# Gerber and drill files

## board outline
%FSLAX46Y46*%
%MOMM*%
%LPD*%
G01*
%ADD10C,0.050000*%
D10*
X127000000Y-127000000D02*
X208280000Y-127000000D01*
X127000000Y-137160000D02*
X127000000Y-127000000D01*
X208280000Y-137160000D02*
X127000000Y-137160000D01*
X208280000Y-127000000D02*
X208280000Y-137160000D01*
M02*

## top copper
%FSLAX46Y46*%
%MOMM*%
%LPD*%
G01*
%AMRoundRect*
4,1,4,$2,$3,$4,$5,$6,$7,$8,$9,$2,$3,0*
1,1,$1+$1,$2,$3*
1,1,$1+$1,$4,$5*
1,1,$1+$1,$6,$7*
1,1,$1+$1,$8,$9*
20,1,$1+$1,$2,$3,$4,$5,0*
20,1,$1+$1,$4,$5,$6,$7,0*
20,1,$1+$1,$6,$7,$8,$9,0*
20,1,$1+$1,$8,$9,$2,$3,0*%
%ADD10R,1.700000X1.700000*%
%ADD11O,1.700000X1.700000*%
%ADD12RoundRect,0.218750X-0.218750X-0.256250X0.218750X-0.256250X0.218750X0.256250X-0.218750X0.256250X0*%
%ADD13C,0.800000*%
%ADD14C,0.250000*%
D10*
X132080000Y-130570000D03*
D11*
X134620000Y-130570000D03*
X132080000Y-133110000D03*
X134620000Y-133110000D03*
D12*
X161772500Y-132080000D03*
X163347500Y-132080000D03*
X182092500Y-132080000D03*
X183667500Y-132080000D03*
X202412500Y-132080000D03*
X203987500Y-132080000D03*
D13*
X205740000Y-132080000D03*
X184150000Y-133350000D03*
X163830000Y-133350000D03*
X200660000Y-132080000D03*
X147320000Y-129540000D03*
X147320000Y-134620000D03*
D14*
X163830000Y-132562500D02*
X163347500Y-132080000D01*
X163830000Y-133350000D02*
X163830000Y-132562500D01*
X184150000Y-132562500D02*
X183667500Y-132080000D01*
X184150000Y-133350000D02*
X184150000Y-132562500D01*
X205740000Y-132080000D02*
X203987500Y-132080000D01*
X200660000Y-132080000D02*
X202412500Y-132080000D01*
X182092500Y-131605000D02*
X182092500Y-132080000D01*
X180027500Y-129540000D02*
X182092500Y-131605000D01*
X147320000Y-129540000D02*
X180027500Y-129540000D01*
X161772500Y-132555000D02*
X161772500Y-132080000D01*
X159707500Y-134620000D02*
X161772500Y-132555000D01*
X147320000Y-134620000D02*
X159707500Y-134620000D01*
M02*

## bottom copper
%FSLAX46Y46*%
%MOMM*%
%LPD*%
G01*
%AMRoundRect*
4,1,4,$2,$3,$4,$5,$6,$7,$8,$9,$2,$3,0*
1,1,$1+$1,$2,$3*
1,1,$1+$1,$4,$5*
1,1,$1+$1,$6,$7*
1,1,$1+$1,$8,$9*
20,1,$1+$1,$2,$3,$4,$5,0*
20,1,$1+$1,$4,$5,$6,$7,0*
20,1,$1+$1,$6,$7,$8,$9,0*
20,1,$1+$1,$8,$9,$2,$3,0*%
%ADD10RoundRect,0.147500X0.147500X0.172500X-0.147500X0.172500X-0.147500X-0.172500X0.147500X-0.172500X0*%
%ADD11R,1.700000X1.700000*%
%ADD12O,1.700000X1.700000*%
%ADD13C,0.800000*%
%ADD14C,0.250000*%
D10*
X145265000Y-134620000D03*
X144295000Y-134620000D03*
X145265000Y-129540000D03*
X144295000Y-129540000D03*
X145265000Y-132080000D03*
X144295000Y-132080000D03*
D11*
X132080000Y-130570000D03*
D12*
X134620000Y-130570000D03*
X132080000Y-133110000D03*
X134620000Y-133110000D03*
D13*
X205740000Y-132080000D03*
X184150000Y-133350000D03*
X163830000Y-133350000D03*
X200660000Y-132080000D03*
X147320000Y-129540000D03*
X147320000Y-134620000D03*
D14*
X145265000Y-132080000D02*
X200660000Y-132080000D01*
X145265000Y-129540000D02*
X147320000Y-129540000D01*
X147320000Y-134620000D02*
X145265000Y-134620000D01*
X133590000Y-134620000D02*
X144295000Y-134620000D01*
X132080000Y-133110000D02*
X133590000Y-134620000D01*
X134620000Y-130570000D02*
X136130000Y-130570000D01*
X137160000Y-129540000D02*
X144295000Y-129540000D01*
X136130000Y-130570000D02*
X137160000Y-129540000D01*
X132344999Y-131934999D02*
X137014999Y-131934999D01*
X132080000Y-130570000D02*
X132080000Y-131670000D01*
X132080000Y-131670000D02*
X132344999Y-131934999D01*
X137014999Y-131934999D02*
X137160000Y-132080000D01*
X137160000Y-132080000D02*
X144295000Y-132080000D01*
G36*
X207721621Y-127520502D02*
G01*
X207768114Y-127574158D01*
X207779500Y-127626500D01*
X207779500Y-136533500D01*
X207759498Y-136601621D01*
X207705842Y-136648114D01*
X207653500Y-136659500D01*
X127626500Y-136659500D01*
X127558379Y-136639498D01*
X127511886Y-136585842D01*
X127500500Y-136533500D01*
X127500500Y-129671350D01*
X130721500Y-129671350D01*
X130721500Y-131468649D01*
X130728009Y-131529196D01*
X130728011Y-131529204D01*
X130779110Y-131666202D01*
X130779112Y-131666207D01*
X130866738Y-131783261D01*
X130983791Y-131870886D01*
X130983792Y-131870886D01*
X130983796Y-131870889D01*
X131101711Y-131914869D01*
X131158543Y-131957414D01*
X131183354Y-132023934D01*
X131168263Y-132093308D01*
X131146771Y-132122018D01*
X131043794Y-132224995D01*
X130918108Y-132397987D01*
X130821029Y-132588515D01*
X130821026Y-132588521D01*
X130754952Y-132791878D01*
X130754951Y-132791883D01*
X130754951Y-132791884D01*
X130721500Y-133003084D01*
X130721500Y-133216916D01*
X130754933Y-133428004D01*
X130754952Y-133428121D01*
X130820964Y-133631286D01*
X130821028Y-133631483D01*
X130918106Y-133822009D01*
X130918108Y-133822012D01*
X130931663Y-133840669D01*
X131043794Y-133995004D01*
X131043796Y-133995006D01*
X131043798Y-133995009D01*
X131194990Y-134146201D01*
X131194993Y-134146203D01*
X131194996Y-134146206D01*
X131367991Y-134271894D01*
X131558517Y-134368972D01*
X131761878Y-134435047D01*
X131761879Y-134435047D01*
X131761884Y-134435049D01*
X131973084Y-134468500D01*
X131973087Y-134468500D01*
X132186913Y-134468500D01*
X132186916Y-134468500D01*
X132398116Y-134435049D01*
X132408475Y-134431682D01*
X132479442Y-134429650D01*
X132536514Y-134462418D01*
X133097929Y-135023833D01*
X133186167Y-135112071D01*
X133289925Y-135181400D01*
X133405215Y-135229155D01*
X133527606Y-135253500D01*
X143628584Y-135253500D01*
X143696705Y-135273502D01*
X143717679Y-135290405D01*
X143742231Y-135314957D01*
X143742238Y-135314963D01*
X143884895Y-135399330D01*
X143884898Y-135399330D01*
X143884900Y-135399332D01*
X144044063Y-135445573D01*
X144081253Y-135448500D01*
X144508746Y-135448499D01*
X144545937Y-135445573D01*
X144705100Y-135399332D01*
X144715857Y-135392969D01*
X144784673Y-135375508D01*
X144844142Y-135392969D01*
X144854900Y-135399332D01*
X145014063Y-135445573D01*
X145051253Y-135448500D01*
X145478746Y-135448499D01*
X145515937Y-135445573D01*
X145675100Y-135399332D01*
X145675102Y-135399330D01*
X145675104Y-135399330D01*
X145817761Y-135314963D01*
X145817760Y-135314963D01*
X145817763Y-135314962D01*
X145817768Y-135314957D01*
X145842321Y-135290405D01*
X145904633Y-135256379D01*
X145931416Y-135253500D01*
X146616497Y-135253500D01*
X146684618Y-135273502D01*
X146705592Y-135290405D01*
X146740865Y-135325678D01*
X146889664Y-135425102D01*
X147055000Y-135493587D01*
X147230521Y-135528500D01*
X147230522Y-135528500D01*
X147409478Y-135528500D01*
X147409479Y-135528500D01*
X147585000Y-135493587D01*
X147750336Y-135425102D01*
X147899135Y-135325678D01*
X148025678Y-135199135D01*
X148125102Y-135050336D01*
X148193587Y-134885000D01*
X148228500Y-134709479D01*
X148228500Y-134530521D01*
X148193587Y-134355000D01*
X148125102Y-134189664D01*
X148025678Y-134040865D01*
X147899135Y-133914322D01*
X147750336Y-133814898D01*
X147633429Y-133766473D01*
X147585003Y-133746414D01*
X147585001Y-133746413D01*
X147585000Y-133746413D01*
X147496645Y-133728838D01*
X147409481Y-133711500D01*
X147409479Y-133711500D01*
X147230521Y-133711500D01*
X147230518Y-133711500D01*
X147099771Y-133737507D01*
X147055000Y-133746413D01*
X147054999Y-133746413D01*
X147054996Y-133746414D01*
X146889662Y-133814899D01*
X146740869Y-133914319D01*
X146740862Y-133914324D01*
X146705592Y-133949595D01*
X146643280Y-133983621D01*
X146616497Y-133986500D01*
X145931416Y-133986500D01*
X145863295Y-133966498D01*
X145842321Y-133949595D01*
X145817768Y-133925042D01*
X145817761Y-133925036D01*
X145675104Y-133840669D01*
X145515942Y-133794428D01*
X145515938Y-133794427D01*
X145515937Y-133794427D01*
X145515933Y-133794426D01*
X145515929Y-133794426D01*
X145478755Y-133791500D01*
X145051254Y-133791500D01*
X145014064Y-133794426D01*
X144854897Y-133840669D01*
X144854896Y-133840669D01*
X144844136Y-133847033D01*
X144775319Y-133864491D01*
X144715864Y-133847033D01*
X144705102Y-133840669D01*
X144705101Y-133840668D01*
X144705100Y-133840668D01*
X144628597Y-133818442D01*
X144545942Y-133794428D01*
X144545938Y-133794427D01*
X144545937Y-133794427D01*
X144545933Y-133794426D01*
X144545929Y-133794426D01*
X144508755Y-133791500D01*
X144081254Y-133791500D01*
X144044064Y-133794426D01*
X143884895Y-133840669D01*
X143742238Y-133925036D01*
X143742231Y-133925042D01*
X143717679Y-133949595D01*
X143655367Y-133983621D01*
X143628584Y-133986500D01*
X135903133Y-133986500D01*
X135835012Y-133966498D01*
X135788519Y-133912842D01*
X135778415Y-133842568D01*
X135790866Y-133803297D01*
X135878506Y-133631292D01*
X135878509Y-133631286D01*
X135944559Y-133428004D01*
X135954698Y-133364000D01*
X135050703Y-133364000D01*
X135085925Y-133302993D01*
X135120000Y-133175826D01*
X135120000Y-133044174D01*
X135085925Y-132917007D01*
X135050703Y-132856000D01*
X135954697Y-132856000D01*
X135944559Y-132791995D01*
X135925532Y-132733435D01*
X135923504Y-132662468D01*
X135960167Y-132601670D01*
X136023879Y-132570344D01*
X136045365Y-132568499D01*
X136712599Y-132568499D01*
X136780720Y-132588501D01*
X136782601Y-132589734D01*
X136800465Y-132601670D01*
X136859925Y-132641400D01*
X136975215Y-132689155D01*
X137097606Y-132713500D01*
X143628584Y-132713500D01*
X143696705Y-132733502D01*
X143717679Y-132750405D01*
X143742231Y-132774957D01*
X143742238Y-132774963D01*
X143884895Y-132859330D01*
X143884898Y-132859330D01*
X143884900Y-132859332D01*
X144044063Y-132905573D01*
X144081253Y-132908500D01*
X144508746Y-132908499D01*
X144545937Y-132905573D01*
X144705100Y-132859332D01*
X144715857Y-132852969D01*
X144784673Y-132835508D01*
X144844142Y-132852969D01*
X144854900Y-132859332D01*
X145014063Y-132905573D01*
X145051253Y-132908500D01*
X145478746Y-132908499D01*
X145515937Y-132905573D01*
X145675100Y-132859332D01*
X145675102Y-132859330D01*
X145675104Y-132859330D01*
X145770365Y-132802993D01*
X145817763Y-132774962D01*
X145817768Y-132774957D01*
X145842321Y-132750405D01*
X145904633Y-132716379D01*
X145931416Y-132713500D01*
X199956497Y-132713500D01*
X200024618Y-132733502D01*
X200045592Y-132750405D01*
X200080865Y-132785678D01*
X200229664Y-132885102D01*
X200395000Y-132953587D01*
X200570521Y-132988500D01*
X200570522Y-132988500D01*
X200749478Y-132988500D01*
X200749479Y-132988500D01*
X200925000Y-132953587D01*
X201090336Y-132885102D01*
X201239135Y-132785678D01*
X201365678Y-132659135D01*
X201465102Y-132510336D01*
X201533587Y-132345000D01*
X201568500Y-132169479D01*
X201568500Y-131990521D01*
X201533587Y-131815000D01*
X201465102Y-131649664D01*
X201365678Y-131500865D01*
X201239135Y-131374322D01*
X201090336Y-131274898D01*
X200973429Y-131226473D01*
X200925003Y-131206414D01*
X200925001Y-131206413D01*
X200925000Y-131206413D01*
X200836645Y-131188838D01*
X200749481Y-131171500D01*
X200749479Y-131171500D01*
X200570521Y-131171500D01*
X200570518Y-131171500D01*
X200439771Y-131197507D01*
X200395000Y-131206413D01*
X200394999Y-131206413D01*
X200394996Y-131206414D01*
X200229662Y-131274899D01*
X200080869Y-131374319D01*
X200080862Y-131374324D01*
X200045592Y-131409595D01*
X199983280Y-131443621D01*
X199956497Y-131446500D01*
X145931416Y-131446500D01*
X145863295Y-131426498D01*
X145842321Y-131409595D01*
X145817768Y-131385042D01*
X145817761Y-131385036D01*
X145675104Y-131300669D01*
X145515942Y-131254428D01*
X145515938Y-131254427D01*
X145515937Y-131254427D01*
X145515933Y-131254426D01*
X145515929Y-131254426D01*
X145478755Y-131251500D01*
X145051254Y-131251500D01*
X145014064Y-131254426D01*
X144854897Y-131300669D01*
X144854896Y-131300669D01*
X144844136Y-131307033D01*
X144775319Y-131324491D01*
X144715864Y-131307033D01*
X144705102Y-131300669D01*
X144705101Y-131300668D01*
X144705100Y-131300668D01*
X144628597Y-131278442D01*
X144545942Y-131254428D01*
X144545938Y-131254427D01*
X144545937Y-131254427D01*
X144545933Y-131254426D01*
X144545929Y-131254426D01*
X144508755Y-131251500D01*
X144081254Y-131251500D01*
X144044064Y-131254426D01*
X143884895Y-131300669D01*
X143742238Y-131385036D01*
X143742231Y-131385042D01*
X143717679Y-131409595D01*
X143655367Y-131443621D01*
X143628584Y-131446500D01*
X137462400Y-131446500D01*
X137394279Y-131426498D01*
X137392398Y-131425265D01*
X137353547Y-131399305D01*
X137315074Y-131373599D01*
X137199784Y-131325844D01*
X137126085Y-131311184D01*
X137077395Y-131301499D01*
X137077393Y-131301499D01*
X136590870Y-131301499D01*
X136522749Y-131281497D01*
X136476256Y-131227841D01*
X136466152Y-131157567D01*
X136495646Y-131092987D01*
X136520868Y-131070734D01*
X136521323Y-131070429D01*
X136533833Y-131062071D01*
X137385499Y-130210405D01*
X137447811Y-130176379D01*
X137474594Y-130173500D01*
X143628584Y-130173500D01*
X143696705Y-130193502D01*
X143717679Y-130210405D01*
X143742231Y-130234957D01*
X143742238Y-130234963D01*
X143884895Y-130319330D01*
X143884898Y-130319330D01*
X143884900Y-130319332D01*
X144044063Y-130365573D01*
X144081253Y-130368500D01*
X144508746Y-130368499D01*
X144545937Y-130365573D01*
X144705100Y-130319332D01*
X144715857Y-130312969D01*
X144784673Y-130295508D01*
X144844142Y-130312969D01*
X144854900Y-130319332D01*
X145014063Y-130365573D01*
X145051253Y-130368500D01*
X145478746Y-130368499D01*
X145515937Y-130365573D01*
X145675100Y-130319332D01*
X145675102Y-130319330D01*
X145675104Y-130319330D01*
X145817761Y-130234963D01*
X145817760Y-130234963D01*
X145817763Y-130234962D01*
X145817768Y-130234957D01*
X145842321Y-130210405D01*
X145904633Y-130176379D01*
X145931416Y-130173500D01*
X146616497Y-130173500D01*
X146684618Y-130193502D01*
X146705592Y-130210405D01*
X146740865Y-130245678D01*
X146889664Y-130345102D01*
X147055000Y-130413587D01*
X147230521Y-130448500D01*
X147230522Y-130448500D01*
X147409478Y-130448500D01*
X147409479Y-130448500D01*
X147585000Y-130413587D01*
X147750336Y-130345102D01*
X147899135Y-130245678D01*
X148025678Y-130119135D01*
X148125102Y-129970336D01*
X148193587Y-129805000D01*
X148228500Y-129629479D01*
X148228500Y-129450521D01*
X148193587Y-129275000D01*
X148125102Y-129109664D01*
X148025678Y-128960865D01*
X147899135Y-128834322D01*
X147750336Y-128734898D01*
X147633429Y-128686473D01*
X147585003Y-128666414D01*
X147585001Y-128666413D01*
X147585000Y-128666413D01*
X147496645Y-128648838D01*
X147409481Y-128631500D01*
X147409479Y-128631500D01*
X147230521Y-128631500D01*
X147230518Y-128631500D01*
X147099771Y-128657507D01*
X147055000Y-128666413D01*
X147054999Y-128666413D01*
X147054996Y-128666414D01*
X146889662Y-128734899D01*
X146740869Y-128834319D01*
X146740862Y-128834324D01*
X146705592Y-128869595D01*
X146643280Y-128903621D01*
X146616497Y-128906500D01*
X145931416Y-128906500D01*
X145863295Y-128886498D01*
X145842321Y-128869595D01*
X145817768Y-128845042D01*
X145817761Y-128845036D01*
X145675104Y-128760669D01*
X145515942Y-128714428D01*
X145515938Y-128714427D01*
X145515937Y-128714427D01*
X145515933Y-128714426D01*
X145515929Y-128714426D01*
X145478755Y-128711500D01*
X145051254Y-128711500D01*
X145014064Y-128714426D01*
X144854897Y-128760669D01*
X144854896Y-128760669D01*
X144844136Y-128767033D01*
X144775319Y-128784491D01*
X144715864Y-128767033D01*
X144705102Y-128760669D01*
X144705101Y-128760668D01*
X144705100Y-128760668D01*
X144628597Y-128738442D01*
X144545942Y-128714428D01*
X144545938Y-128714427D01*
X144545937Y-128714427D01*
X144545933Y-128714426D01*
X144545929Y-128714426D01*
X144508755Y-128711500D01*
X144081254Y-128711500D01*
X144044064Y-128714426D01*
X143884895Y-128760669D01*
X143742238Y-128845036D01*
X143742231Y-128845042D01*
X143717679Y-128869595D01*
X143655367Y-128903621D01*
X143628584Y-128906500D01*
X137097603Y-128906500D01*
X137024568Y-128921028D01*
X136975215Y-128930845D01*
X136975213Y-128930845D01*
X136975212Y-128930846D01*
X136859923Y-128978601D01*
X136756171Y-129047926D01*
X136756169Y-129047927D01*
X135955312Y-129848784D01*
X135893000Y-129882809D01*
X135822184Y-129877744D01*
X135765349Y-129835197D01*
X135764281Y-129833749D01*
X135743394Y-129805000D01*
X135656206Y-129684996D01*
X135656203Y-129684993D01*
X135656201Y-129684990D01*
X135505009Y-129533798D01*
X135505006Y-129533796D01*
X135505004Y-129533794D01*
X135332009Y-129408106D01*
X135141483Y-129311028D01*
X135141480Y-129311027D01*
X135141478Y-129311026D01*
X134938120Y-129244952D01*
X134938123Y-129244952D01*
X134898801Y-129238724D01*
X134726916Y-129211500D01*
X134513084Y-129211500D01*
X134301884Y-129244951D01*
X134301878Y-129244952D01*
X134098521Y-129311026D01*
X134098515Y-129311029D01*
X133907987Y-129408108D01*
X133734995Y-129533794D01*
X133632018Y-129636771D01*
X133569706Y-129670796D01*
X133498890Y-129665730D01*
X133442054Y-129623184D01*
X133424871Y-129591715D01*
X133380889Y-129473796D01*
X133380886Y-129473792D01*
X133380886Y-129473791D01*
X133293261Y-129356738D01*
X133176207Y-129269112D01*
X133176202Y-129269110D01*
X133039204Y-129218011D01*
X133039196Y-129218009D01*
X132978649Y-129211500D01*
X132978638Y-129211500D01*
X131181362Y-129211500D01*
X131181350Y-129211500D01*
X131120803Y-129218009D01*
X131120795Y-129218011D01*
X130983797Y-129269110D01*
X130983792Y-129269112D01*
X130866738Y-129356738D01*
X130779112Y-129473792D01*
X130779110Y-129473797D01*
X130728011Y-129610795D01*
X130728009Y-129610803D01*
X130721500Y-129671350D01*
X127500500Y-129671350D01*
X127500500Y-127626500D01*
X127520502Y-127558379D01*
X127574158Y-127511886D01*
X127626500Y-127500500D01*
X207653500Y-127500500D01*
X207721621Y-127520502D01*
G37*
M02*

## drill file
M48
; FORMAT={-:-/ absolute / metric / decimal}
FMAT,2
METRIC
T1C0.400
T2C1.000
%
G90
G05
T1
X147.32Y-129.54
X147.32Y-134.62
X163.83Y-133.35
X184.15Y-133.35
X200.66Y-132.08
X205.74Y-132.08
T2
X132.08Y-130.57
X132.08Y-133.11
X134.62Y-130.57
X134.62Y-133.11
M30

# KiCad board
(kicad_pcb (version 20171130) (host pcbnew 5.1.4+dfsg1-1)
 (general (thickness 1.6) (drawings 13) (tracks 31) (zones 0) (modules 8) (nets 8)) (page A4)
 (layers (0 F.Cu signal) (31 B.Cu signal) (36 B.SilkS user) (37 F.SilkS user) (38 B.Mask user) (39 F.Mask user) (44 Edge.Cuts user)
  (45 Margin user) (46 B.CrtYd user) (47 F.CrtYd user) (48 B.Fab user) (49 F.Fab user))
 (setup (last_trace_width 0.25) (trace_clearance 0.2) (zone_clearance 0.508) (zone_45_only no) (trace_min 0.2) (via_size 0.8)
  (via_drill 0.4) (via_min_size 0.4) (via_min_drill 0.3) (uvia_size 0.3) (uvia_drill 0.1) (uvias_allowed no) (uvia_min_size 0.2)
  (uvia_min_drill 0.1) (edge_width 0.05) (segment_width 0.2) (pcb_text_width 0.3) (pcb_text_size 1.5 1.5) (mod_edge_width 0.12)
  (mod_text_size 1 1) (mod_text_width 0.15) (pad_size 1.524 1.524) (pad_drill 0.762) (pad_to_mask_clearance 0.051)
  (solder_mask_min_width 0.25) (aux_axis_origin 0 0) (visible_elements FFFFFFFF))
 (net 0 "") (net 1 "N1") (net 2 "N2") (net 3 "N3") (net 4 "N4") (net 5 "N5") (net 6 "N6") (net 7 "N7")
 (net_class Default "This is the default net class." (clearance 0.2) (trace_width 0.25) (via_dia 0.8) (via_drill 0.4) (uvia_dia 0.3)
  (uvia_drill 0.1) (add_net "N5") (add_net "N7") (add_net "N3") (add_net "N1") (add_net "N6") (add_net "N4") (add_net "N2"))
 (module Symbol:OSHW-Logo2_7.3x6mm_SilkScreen (layer B.Cu) (at 191.77 132.08 180)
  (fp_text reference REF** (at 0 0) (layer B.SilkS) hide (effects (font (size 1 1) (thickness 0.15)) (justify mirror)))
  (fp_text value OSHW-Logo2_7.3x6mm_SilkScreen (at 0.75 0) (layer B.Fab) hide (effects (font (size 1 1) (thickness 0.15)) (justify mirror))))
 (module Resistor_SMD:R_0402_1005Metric (layer B.Cu) (at 144.78 134.62 180)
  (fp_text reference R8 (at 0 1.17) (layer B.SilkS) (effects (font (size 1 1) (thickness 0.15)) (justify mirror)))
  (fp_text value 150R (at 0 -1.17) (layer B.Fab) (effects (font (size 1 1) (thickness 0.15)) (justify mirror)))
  (pad 1 smd roundrect (at -0.485 0 180) (size 0.59 0.64) (layers B.Cu B.Paste B.Mask) (roundrect_rratio 0.25) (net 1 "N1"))
  (pad 2 smd roundrect (at 0.485 0 180) (size 0.59 0.64) (layers B.Cu B.Paste B.Mask) (roundrect_rratio 0.25) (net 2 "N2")))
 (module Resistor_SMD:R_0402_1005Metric (layer B.Cu) (at 144.78 129.54 180)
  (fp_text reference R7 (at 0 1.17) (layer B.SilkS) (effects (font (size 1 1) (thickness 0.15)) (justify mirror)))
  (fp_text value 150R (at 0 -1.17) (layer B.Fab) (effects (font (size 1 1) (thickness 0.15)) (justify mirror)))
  (pad 1 smd roundrect (at -0.485 0 180) (size 0.59 0.64) (layers B.Cu B.Paste B.Mask) (roundrect_rratio 0.25) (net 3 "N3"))
  (pad 2 smd roundrect (at 0.485 0 180) (size 0.59 0.64) (layers B.Cu B.Paste B.Mask) (roundrect_rratio 0.25) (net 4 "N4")))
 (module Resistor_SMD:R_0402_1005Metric (layer B.Cu) (at 144.78 132.08 180)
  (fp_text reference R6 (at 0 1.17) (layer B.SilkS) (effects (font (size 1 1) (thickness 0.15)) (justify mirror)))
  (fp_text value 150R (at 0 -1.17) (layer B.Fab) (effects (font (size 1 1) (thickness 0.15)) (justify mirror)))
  (pad 1 smd roundrect (at -0.485 0 180) (size 0.59 0.64) (layers B.Cu B.Paste B.Mask) (roundrect_rratio 0.25) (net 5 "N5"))
  (pad 2 smd roundrect (at 0.485 0 180) (size 0.59 0.64) (layers B.Cu B.Paste B.Mask) (roundrect_rratio 0.25) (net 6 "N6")))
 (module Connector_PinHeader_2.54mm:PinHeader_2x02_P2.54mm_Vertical (layer F.Cu) (at 132.08 130.57)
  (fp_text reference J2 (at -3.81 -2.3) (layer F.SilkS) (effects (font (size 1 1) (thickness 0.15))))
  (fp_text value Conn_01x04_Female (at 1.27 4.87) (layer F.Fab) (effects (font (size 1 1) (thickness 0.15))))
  (pad 1 thru_hole rect (at 0 0) (size 1.7 1.7) (drill 1) (layers *.Cu *.Mask) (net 6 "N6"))
  (pad 2 thru_hole oval (at 2.54 0) (size 1.7 1.7) (drill 1) (layers *.Cu *.Mask) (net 4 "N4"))
  (pad 3 thru_hole oval (at 0 2.54) (size 1.7 1.7) (drill 1) (layers *.Cu *.Mask) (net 2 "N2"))
  (pad 4 thru_hole oval (at 2.54 2.54) (size 1.7 1.7) (drill 1) (layers *.Cu *.Mask) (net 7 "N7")))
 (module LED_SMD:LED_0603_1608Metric (layer F.Cu) (at 162.56 132.08)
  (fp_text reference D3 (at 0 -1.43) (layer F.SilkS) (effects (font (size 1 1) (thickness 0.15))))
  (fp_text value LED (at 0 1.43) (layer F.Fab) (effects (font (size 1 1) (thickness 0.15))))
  (pad 1 smd roundrect (at -0.7875 0) (size 0.875 0.95) (layers F.Cu F.Paste F.Mask) (roundrect_rratio 0.25) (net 1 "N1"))
  (pad 2 smd roundrect (at 0.7875 0) (size 0.875 0.95) (layers F.Cu F.Paste F.Mask) (roundrect_rratio 0.25) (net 7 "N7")))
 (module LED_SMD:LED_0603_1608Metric (layer F.Cu) (at 182.88 132.08)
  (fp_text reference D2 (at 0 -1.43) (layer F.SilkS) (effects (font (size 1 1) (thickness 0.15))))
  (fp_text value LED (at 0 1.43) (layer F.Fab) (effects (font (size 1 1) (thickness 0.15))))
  (pad 1 smd roundrect (at -0.7875 0) (size 0.875 0.95) (layers F.Cu F.Paste F.Mask) (roundrect_rratio 0.25) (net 3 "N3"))
  (pad 2 smd roundrect (at 0.7875 0) (size 0.875 0.95) (layers F.Cu F.Paste F.Mask) (roundrect_rratio 0.25) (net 7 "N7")))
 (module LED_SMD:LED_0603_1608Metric (layer F.Cu) (at 203.2 132.08)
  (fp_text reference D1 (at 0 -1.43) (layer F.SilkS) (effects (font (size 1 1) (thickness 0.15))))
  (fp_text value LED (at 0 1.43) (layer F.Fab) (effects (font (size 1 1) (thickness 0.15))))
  (pad 1 smd roundrect (at -0.7875 0) (size 0.875 0.95) (layers F.Cu F.Paste F.Mask) (roundrect_rratio 0.25) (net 5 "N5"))
  (pad 2 smd roundrect (at 0.7875 0) (size 0.875 0.95) (layers F.Cu F.Paste F.Mask) (roundrect_rratio 0.25) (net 7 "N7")))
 (gr_line (start 127 127) (end 208.28 127) (layer Edge.Cuts) (width 0.05))
 (gr_line (start 127 137.16) (end 127 127) (layer Edge.Cuts) (width 0.05))
 (gr_line (start 208.28 137.16) (end 127 137.16) (layer Edge.Cuts) (width 0.05))
 (gr_line (start 208.28 127) (end 208.28 137.16) (layer Edge.Cuts) (width 0.05))
 (via (at 205.74 132.08) (size 0.8) (drill 0.4) (layers F.Cu B.Cu) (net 7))
 (via (at 184.15 133.35) (size 0.8) (drill 0.4) (layers F.Cu B.Cu) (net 7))
 (via (at 163.83 133.35) (size 0.8) (drill 0.4) (layers F.Cu B.Cu) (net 7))
 (segment (start 163.83 132.5625) (end 163.3475 132.08) (width 0.25) (layer F.Cu) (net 7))
 (segment (start 163.83 133.35) (end 163.83 132.5625) (width 0.25) (layer F.Cu) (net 7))
 (segment (start 184.15 132.5625) (end 183.6675 132.08) (width 0.25) (layer F.Cu) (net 7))
 (segment (start 184.15 133.35) (end 184.15 132.5625) (width 0.25) (layer F.Cu) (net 7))
 (segment (start 205.74 132.08) (end 203.9875 132.08) (width 0.25) (layer F.Cu) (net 7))
 (via (at 200.66 132.08) (size 0.8) (drill 0.4) (layers F.Cu B.Cu) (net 5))
 (segment (start 145.265 132.08) (end 200.66 132.08) (width 0.25) (layer B.Cu) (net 5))
 (segment (start 200.66 132.08) (end 202.4125 132.08) (width 0.25) (layer F.Cu) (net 5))
 (via (at 147.32 129.54) (size 0.8) (drill 0.4) (layers F.Cu B.Cu) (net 3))
 (segment (start 182.0925 131.605) (end 182.0925 132.08) (width 0.25) (layer F.Cu) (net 3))
 (segment (start 180.0275 129.54) (end 182.0925 131.605) (width 0.25) (layer F.Cu) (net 3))
 (segment (start 147.32 129.54) (end 180.0275 129.54) (width 0.25) (layer F.Cu) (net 3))
 (segment (start 145.265 129.54) (end 147.32 129.54) (width 0.25) (layer B.Cu) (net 3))
 (via (at 147.32 134.62) (size 0.8) (drill 0.4) (layers F.Cu B.Cu) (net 1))
 (segment (start 147.32 134.62) (end 145.265 134.62) (width 0.25) (layer B.Cu) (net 1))
 (segment (start 161.7725 132.555) (end 161.7725 132.08) (width 0.25) (layer F.Cu) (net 1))
 (segment (start 159.7075 134.62) (end 161.7725 132.555) (width 0.25) (layer F.Cu) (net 1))
 (segment (start 147.32 134.62) (end 159.7075 134.62) (width 0.25) (layer F.Cu) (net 1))
 (segment (start 133.59 134.62) (end 144.295 134.62) (width 0.25) (layer B.Cu) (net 2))
 (segment (start 132.08 133.11) (end 133.59 134.62) (width 0.25) (layer B.Cu) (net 2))
 (segment (start 134.62 130.57) (end 136.13 130.57) (width 0.25) (layer B.Cu) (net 4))
 (segment (start 137.16 129.54) (end 144.295 129.54) (width 0.25) (layer B.Cu) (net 4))
 (segment (start 136.13 130.57) (end 137.16 129.54) (width 0.25) (layer B.Cu) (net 4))
 (segment (start 132.344999 131.934999) (end 137.014999 131.934999) (width 0.25) (layer B.Cu) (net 6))
 (segment (start 132.08 130.57) (end 132.08 131.67) (width 0.25) (layer B.Cu) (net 6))
 (segment (start 132.08 131.67) (end 132.344999 131.934999) (width 0.25) (layer B.Cu) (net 6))
 (segment (start 137.014999 131.934999) (end 137.16 132.08) (width 0.25) (layer B.Cu) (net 6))
 (segment (start 137.16 132.08) (end 144.295 132.08) (width 0.25) (layer B.Cu) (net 6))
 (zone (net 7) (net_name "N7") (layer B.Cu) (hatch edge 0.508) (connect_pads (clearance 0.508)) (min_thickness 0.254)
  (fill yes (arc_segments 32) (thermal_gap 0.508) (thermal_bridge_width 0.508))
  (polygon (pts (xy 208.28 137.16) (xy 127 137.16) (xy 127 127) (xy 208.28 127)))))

